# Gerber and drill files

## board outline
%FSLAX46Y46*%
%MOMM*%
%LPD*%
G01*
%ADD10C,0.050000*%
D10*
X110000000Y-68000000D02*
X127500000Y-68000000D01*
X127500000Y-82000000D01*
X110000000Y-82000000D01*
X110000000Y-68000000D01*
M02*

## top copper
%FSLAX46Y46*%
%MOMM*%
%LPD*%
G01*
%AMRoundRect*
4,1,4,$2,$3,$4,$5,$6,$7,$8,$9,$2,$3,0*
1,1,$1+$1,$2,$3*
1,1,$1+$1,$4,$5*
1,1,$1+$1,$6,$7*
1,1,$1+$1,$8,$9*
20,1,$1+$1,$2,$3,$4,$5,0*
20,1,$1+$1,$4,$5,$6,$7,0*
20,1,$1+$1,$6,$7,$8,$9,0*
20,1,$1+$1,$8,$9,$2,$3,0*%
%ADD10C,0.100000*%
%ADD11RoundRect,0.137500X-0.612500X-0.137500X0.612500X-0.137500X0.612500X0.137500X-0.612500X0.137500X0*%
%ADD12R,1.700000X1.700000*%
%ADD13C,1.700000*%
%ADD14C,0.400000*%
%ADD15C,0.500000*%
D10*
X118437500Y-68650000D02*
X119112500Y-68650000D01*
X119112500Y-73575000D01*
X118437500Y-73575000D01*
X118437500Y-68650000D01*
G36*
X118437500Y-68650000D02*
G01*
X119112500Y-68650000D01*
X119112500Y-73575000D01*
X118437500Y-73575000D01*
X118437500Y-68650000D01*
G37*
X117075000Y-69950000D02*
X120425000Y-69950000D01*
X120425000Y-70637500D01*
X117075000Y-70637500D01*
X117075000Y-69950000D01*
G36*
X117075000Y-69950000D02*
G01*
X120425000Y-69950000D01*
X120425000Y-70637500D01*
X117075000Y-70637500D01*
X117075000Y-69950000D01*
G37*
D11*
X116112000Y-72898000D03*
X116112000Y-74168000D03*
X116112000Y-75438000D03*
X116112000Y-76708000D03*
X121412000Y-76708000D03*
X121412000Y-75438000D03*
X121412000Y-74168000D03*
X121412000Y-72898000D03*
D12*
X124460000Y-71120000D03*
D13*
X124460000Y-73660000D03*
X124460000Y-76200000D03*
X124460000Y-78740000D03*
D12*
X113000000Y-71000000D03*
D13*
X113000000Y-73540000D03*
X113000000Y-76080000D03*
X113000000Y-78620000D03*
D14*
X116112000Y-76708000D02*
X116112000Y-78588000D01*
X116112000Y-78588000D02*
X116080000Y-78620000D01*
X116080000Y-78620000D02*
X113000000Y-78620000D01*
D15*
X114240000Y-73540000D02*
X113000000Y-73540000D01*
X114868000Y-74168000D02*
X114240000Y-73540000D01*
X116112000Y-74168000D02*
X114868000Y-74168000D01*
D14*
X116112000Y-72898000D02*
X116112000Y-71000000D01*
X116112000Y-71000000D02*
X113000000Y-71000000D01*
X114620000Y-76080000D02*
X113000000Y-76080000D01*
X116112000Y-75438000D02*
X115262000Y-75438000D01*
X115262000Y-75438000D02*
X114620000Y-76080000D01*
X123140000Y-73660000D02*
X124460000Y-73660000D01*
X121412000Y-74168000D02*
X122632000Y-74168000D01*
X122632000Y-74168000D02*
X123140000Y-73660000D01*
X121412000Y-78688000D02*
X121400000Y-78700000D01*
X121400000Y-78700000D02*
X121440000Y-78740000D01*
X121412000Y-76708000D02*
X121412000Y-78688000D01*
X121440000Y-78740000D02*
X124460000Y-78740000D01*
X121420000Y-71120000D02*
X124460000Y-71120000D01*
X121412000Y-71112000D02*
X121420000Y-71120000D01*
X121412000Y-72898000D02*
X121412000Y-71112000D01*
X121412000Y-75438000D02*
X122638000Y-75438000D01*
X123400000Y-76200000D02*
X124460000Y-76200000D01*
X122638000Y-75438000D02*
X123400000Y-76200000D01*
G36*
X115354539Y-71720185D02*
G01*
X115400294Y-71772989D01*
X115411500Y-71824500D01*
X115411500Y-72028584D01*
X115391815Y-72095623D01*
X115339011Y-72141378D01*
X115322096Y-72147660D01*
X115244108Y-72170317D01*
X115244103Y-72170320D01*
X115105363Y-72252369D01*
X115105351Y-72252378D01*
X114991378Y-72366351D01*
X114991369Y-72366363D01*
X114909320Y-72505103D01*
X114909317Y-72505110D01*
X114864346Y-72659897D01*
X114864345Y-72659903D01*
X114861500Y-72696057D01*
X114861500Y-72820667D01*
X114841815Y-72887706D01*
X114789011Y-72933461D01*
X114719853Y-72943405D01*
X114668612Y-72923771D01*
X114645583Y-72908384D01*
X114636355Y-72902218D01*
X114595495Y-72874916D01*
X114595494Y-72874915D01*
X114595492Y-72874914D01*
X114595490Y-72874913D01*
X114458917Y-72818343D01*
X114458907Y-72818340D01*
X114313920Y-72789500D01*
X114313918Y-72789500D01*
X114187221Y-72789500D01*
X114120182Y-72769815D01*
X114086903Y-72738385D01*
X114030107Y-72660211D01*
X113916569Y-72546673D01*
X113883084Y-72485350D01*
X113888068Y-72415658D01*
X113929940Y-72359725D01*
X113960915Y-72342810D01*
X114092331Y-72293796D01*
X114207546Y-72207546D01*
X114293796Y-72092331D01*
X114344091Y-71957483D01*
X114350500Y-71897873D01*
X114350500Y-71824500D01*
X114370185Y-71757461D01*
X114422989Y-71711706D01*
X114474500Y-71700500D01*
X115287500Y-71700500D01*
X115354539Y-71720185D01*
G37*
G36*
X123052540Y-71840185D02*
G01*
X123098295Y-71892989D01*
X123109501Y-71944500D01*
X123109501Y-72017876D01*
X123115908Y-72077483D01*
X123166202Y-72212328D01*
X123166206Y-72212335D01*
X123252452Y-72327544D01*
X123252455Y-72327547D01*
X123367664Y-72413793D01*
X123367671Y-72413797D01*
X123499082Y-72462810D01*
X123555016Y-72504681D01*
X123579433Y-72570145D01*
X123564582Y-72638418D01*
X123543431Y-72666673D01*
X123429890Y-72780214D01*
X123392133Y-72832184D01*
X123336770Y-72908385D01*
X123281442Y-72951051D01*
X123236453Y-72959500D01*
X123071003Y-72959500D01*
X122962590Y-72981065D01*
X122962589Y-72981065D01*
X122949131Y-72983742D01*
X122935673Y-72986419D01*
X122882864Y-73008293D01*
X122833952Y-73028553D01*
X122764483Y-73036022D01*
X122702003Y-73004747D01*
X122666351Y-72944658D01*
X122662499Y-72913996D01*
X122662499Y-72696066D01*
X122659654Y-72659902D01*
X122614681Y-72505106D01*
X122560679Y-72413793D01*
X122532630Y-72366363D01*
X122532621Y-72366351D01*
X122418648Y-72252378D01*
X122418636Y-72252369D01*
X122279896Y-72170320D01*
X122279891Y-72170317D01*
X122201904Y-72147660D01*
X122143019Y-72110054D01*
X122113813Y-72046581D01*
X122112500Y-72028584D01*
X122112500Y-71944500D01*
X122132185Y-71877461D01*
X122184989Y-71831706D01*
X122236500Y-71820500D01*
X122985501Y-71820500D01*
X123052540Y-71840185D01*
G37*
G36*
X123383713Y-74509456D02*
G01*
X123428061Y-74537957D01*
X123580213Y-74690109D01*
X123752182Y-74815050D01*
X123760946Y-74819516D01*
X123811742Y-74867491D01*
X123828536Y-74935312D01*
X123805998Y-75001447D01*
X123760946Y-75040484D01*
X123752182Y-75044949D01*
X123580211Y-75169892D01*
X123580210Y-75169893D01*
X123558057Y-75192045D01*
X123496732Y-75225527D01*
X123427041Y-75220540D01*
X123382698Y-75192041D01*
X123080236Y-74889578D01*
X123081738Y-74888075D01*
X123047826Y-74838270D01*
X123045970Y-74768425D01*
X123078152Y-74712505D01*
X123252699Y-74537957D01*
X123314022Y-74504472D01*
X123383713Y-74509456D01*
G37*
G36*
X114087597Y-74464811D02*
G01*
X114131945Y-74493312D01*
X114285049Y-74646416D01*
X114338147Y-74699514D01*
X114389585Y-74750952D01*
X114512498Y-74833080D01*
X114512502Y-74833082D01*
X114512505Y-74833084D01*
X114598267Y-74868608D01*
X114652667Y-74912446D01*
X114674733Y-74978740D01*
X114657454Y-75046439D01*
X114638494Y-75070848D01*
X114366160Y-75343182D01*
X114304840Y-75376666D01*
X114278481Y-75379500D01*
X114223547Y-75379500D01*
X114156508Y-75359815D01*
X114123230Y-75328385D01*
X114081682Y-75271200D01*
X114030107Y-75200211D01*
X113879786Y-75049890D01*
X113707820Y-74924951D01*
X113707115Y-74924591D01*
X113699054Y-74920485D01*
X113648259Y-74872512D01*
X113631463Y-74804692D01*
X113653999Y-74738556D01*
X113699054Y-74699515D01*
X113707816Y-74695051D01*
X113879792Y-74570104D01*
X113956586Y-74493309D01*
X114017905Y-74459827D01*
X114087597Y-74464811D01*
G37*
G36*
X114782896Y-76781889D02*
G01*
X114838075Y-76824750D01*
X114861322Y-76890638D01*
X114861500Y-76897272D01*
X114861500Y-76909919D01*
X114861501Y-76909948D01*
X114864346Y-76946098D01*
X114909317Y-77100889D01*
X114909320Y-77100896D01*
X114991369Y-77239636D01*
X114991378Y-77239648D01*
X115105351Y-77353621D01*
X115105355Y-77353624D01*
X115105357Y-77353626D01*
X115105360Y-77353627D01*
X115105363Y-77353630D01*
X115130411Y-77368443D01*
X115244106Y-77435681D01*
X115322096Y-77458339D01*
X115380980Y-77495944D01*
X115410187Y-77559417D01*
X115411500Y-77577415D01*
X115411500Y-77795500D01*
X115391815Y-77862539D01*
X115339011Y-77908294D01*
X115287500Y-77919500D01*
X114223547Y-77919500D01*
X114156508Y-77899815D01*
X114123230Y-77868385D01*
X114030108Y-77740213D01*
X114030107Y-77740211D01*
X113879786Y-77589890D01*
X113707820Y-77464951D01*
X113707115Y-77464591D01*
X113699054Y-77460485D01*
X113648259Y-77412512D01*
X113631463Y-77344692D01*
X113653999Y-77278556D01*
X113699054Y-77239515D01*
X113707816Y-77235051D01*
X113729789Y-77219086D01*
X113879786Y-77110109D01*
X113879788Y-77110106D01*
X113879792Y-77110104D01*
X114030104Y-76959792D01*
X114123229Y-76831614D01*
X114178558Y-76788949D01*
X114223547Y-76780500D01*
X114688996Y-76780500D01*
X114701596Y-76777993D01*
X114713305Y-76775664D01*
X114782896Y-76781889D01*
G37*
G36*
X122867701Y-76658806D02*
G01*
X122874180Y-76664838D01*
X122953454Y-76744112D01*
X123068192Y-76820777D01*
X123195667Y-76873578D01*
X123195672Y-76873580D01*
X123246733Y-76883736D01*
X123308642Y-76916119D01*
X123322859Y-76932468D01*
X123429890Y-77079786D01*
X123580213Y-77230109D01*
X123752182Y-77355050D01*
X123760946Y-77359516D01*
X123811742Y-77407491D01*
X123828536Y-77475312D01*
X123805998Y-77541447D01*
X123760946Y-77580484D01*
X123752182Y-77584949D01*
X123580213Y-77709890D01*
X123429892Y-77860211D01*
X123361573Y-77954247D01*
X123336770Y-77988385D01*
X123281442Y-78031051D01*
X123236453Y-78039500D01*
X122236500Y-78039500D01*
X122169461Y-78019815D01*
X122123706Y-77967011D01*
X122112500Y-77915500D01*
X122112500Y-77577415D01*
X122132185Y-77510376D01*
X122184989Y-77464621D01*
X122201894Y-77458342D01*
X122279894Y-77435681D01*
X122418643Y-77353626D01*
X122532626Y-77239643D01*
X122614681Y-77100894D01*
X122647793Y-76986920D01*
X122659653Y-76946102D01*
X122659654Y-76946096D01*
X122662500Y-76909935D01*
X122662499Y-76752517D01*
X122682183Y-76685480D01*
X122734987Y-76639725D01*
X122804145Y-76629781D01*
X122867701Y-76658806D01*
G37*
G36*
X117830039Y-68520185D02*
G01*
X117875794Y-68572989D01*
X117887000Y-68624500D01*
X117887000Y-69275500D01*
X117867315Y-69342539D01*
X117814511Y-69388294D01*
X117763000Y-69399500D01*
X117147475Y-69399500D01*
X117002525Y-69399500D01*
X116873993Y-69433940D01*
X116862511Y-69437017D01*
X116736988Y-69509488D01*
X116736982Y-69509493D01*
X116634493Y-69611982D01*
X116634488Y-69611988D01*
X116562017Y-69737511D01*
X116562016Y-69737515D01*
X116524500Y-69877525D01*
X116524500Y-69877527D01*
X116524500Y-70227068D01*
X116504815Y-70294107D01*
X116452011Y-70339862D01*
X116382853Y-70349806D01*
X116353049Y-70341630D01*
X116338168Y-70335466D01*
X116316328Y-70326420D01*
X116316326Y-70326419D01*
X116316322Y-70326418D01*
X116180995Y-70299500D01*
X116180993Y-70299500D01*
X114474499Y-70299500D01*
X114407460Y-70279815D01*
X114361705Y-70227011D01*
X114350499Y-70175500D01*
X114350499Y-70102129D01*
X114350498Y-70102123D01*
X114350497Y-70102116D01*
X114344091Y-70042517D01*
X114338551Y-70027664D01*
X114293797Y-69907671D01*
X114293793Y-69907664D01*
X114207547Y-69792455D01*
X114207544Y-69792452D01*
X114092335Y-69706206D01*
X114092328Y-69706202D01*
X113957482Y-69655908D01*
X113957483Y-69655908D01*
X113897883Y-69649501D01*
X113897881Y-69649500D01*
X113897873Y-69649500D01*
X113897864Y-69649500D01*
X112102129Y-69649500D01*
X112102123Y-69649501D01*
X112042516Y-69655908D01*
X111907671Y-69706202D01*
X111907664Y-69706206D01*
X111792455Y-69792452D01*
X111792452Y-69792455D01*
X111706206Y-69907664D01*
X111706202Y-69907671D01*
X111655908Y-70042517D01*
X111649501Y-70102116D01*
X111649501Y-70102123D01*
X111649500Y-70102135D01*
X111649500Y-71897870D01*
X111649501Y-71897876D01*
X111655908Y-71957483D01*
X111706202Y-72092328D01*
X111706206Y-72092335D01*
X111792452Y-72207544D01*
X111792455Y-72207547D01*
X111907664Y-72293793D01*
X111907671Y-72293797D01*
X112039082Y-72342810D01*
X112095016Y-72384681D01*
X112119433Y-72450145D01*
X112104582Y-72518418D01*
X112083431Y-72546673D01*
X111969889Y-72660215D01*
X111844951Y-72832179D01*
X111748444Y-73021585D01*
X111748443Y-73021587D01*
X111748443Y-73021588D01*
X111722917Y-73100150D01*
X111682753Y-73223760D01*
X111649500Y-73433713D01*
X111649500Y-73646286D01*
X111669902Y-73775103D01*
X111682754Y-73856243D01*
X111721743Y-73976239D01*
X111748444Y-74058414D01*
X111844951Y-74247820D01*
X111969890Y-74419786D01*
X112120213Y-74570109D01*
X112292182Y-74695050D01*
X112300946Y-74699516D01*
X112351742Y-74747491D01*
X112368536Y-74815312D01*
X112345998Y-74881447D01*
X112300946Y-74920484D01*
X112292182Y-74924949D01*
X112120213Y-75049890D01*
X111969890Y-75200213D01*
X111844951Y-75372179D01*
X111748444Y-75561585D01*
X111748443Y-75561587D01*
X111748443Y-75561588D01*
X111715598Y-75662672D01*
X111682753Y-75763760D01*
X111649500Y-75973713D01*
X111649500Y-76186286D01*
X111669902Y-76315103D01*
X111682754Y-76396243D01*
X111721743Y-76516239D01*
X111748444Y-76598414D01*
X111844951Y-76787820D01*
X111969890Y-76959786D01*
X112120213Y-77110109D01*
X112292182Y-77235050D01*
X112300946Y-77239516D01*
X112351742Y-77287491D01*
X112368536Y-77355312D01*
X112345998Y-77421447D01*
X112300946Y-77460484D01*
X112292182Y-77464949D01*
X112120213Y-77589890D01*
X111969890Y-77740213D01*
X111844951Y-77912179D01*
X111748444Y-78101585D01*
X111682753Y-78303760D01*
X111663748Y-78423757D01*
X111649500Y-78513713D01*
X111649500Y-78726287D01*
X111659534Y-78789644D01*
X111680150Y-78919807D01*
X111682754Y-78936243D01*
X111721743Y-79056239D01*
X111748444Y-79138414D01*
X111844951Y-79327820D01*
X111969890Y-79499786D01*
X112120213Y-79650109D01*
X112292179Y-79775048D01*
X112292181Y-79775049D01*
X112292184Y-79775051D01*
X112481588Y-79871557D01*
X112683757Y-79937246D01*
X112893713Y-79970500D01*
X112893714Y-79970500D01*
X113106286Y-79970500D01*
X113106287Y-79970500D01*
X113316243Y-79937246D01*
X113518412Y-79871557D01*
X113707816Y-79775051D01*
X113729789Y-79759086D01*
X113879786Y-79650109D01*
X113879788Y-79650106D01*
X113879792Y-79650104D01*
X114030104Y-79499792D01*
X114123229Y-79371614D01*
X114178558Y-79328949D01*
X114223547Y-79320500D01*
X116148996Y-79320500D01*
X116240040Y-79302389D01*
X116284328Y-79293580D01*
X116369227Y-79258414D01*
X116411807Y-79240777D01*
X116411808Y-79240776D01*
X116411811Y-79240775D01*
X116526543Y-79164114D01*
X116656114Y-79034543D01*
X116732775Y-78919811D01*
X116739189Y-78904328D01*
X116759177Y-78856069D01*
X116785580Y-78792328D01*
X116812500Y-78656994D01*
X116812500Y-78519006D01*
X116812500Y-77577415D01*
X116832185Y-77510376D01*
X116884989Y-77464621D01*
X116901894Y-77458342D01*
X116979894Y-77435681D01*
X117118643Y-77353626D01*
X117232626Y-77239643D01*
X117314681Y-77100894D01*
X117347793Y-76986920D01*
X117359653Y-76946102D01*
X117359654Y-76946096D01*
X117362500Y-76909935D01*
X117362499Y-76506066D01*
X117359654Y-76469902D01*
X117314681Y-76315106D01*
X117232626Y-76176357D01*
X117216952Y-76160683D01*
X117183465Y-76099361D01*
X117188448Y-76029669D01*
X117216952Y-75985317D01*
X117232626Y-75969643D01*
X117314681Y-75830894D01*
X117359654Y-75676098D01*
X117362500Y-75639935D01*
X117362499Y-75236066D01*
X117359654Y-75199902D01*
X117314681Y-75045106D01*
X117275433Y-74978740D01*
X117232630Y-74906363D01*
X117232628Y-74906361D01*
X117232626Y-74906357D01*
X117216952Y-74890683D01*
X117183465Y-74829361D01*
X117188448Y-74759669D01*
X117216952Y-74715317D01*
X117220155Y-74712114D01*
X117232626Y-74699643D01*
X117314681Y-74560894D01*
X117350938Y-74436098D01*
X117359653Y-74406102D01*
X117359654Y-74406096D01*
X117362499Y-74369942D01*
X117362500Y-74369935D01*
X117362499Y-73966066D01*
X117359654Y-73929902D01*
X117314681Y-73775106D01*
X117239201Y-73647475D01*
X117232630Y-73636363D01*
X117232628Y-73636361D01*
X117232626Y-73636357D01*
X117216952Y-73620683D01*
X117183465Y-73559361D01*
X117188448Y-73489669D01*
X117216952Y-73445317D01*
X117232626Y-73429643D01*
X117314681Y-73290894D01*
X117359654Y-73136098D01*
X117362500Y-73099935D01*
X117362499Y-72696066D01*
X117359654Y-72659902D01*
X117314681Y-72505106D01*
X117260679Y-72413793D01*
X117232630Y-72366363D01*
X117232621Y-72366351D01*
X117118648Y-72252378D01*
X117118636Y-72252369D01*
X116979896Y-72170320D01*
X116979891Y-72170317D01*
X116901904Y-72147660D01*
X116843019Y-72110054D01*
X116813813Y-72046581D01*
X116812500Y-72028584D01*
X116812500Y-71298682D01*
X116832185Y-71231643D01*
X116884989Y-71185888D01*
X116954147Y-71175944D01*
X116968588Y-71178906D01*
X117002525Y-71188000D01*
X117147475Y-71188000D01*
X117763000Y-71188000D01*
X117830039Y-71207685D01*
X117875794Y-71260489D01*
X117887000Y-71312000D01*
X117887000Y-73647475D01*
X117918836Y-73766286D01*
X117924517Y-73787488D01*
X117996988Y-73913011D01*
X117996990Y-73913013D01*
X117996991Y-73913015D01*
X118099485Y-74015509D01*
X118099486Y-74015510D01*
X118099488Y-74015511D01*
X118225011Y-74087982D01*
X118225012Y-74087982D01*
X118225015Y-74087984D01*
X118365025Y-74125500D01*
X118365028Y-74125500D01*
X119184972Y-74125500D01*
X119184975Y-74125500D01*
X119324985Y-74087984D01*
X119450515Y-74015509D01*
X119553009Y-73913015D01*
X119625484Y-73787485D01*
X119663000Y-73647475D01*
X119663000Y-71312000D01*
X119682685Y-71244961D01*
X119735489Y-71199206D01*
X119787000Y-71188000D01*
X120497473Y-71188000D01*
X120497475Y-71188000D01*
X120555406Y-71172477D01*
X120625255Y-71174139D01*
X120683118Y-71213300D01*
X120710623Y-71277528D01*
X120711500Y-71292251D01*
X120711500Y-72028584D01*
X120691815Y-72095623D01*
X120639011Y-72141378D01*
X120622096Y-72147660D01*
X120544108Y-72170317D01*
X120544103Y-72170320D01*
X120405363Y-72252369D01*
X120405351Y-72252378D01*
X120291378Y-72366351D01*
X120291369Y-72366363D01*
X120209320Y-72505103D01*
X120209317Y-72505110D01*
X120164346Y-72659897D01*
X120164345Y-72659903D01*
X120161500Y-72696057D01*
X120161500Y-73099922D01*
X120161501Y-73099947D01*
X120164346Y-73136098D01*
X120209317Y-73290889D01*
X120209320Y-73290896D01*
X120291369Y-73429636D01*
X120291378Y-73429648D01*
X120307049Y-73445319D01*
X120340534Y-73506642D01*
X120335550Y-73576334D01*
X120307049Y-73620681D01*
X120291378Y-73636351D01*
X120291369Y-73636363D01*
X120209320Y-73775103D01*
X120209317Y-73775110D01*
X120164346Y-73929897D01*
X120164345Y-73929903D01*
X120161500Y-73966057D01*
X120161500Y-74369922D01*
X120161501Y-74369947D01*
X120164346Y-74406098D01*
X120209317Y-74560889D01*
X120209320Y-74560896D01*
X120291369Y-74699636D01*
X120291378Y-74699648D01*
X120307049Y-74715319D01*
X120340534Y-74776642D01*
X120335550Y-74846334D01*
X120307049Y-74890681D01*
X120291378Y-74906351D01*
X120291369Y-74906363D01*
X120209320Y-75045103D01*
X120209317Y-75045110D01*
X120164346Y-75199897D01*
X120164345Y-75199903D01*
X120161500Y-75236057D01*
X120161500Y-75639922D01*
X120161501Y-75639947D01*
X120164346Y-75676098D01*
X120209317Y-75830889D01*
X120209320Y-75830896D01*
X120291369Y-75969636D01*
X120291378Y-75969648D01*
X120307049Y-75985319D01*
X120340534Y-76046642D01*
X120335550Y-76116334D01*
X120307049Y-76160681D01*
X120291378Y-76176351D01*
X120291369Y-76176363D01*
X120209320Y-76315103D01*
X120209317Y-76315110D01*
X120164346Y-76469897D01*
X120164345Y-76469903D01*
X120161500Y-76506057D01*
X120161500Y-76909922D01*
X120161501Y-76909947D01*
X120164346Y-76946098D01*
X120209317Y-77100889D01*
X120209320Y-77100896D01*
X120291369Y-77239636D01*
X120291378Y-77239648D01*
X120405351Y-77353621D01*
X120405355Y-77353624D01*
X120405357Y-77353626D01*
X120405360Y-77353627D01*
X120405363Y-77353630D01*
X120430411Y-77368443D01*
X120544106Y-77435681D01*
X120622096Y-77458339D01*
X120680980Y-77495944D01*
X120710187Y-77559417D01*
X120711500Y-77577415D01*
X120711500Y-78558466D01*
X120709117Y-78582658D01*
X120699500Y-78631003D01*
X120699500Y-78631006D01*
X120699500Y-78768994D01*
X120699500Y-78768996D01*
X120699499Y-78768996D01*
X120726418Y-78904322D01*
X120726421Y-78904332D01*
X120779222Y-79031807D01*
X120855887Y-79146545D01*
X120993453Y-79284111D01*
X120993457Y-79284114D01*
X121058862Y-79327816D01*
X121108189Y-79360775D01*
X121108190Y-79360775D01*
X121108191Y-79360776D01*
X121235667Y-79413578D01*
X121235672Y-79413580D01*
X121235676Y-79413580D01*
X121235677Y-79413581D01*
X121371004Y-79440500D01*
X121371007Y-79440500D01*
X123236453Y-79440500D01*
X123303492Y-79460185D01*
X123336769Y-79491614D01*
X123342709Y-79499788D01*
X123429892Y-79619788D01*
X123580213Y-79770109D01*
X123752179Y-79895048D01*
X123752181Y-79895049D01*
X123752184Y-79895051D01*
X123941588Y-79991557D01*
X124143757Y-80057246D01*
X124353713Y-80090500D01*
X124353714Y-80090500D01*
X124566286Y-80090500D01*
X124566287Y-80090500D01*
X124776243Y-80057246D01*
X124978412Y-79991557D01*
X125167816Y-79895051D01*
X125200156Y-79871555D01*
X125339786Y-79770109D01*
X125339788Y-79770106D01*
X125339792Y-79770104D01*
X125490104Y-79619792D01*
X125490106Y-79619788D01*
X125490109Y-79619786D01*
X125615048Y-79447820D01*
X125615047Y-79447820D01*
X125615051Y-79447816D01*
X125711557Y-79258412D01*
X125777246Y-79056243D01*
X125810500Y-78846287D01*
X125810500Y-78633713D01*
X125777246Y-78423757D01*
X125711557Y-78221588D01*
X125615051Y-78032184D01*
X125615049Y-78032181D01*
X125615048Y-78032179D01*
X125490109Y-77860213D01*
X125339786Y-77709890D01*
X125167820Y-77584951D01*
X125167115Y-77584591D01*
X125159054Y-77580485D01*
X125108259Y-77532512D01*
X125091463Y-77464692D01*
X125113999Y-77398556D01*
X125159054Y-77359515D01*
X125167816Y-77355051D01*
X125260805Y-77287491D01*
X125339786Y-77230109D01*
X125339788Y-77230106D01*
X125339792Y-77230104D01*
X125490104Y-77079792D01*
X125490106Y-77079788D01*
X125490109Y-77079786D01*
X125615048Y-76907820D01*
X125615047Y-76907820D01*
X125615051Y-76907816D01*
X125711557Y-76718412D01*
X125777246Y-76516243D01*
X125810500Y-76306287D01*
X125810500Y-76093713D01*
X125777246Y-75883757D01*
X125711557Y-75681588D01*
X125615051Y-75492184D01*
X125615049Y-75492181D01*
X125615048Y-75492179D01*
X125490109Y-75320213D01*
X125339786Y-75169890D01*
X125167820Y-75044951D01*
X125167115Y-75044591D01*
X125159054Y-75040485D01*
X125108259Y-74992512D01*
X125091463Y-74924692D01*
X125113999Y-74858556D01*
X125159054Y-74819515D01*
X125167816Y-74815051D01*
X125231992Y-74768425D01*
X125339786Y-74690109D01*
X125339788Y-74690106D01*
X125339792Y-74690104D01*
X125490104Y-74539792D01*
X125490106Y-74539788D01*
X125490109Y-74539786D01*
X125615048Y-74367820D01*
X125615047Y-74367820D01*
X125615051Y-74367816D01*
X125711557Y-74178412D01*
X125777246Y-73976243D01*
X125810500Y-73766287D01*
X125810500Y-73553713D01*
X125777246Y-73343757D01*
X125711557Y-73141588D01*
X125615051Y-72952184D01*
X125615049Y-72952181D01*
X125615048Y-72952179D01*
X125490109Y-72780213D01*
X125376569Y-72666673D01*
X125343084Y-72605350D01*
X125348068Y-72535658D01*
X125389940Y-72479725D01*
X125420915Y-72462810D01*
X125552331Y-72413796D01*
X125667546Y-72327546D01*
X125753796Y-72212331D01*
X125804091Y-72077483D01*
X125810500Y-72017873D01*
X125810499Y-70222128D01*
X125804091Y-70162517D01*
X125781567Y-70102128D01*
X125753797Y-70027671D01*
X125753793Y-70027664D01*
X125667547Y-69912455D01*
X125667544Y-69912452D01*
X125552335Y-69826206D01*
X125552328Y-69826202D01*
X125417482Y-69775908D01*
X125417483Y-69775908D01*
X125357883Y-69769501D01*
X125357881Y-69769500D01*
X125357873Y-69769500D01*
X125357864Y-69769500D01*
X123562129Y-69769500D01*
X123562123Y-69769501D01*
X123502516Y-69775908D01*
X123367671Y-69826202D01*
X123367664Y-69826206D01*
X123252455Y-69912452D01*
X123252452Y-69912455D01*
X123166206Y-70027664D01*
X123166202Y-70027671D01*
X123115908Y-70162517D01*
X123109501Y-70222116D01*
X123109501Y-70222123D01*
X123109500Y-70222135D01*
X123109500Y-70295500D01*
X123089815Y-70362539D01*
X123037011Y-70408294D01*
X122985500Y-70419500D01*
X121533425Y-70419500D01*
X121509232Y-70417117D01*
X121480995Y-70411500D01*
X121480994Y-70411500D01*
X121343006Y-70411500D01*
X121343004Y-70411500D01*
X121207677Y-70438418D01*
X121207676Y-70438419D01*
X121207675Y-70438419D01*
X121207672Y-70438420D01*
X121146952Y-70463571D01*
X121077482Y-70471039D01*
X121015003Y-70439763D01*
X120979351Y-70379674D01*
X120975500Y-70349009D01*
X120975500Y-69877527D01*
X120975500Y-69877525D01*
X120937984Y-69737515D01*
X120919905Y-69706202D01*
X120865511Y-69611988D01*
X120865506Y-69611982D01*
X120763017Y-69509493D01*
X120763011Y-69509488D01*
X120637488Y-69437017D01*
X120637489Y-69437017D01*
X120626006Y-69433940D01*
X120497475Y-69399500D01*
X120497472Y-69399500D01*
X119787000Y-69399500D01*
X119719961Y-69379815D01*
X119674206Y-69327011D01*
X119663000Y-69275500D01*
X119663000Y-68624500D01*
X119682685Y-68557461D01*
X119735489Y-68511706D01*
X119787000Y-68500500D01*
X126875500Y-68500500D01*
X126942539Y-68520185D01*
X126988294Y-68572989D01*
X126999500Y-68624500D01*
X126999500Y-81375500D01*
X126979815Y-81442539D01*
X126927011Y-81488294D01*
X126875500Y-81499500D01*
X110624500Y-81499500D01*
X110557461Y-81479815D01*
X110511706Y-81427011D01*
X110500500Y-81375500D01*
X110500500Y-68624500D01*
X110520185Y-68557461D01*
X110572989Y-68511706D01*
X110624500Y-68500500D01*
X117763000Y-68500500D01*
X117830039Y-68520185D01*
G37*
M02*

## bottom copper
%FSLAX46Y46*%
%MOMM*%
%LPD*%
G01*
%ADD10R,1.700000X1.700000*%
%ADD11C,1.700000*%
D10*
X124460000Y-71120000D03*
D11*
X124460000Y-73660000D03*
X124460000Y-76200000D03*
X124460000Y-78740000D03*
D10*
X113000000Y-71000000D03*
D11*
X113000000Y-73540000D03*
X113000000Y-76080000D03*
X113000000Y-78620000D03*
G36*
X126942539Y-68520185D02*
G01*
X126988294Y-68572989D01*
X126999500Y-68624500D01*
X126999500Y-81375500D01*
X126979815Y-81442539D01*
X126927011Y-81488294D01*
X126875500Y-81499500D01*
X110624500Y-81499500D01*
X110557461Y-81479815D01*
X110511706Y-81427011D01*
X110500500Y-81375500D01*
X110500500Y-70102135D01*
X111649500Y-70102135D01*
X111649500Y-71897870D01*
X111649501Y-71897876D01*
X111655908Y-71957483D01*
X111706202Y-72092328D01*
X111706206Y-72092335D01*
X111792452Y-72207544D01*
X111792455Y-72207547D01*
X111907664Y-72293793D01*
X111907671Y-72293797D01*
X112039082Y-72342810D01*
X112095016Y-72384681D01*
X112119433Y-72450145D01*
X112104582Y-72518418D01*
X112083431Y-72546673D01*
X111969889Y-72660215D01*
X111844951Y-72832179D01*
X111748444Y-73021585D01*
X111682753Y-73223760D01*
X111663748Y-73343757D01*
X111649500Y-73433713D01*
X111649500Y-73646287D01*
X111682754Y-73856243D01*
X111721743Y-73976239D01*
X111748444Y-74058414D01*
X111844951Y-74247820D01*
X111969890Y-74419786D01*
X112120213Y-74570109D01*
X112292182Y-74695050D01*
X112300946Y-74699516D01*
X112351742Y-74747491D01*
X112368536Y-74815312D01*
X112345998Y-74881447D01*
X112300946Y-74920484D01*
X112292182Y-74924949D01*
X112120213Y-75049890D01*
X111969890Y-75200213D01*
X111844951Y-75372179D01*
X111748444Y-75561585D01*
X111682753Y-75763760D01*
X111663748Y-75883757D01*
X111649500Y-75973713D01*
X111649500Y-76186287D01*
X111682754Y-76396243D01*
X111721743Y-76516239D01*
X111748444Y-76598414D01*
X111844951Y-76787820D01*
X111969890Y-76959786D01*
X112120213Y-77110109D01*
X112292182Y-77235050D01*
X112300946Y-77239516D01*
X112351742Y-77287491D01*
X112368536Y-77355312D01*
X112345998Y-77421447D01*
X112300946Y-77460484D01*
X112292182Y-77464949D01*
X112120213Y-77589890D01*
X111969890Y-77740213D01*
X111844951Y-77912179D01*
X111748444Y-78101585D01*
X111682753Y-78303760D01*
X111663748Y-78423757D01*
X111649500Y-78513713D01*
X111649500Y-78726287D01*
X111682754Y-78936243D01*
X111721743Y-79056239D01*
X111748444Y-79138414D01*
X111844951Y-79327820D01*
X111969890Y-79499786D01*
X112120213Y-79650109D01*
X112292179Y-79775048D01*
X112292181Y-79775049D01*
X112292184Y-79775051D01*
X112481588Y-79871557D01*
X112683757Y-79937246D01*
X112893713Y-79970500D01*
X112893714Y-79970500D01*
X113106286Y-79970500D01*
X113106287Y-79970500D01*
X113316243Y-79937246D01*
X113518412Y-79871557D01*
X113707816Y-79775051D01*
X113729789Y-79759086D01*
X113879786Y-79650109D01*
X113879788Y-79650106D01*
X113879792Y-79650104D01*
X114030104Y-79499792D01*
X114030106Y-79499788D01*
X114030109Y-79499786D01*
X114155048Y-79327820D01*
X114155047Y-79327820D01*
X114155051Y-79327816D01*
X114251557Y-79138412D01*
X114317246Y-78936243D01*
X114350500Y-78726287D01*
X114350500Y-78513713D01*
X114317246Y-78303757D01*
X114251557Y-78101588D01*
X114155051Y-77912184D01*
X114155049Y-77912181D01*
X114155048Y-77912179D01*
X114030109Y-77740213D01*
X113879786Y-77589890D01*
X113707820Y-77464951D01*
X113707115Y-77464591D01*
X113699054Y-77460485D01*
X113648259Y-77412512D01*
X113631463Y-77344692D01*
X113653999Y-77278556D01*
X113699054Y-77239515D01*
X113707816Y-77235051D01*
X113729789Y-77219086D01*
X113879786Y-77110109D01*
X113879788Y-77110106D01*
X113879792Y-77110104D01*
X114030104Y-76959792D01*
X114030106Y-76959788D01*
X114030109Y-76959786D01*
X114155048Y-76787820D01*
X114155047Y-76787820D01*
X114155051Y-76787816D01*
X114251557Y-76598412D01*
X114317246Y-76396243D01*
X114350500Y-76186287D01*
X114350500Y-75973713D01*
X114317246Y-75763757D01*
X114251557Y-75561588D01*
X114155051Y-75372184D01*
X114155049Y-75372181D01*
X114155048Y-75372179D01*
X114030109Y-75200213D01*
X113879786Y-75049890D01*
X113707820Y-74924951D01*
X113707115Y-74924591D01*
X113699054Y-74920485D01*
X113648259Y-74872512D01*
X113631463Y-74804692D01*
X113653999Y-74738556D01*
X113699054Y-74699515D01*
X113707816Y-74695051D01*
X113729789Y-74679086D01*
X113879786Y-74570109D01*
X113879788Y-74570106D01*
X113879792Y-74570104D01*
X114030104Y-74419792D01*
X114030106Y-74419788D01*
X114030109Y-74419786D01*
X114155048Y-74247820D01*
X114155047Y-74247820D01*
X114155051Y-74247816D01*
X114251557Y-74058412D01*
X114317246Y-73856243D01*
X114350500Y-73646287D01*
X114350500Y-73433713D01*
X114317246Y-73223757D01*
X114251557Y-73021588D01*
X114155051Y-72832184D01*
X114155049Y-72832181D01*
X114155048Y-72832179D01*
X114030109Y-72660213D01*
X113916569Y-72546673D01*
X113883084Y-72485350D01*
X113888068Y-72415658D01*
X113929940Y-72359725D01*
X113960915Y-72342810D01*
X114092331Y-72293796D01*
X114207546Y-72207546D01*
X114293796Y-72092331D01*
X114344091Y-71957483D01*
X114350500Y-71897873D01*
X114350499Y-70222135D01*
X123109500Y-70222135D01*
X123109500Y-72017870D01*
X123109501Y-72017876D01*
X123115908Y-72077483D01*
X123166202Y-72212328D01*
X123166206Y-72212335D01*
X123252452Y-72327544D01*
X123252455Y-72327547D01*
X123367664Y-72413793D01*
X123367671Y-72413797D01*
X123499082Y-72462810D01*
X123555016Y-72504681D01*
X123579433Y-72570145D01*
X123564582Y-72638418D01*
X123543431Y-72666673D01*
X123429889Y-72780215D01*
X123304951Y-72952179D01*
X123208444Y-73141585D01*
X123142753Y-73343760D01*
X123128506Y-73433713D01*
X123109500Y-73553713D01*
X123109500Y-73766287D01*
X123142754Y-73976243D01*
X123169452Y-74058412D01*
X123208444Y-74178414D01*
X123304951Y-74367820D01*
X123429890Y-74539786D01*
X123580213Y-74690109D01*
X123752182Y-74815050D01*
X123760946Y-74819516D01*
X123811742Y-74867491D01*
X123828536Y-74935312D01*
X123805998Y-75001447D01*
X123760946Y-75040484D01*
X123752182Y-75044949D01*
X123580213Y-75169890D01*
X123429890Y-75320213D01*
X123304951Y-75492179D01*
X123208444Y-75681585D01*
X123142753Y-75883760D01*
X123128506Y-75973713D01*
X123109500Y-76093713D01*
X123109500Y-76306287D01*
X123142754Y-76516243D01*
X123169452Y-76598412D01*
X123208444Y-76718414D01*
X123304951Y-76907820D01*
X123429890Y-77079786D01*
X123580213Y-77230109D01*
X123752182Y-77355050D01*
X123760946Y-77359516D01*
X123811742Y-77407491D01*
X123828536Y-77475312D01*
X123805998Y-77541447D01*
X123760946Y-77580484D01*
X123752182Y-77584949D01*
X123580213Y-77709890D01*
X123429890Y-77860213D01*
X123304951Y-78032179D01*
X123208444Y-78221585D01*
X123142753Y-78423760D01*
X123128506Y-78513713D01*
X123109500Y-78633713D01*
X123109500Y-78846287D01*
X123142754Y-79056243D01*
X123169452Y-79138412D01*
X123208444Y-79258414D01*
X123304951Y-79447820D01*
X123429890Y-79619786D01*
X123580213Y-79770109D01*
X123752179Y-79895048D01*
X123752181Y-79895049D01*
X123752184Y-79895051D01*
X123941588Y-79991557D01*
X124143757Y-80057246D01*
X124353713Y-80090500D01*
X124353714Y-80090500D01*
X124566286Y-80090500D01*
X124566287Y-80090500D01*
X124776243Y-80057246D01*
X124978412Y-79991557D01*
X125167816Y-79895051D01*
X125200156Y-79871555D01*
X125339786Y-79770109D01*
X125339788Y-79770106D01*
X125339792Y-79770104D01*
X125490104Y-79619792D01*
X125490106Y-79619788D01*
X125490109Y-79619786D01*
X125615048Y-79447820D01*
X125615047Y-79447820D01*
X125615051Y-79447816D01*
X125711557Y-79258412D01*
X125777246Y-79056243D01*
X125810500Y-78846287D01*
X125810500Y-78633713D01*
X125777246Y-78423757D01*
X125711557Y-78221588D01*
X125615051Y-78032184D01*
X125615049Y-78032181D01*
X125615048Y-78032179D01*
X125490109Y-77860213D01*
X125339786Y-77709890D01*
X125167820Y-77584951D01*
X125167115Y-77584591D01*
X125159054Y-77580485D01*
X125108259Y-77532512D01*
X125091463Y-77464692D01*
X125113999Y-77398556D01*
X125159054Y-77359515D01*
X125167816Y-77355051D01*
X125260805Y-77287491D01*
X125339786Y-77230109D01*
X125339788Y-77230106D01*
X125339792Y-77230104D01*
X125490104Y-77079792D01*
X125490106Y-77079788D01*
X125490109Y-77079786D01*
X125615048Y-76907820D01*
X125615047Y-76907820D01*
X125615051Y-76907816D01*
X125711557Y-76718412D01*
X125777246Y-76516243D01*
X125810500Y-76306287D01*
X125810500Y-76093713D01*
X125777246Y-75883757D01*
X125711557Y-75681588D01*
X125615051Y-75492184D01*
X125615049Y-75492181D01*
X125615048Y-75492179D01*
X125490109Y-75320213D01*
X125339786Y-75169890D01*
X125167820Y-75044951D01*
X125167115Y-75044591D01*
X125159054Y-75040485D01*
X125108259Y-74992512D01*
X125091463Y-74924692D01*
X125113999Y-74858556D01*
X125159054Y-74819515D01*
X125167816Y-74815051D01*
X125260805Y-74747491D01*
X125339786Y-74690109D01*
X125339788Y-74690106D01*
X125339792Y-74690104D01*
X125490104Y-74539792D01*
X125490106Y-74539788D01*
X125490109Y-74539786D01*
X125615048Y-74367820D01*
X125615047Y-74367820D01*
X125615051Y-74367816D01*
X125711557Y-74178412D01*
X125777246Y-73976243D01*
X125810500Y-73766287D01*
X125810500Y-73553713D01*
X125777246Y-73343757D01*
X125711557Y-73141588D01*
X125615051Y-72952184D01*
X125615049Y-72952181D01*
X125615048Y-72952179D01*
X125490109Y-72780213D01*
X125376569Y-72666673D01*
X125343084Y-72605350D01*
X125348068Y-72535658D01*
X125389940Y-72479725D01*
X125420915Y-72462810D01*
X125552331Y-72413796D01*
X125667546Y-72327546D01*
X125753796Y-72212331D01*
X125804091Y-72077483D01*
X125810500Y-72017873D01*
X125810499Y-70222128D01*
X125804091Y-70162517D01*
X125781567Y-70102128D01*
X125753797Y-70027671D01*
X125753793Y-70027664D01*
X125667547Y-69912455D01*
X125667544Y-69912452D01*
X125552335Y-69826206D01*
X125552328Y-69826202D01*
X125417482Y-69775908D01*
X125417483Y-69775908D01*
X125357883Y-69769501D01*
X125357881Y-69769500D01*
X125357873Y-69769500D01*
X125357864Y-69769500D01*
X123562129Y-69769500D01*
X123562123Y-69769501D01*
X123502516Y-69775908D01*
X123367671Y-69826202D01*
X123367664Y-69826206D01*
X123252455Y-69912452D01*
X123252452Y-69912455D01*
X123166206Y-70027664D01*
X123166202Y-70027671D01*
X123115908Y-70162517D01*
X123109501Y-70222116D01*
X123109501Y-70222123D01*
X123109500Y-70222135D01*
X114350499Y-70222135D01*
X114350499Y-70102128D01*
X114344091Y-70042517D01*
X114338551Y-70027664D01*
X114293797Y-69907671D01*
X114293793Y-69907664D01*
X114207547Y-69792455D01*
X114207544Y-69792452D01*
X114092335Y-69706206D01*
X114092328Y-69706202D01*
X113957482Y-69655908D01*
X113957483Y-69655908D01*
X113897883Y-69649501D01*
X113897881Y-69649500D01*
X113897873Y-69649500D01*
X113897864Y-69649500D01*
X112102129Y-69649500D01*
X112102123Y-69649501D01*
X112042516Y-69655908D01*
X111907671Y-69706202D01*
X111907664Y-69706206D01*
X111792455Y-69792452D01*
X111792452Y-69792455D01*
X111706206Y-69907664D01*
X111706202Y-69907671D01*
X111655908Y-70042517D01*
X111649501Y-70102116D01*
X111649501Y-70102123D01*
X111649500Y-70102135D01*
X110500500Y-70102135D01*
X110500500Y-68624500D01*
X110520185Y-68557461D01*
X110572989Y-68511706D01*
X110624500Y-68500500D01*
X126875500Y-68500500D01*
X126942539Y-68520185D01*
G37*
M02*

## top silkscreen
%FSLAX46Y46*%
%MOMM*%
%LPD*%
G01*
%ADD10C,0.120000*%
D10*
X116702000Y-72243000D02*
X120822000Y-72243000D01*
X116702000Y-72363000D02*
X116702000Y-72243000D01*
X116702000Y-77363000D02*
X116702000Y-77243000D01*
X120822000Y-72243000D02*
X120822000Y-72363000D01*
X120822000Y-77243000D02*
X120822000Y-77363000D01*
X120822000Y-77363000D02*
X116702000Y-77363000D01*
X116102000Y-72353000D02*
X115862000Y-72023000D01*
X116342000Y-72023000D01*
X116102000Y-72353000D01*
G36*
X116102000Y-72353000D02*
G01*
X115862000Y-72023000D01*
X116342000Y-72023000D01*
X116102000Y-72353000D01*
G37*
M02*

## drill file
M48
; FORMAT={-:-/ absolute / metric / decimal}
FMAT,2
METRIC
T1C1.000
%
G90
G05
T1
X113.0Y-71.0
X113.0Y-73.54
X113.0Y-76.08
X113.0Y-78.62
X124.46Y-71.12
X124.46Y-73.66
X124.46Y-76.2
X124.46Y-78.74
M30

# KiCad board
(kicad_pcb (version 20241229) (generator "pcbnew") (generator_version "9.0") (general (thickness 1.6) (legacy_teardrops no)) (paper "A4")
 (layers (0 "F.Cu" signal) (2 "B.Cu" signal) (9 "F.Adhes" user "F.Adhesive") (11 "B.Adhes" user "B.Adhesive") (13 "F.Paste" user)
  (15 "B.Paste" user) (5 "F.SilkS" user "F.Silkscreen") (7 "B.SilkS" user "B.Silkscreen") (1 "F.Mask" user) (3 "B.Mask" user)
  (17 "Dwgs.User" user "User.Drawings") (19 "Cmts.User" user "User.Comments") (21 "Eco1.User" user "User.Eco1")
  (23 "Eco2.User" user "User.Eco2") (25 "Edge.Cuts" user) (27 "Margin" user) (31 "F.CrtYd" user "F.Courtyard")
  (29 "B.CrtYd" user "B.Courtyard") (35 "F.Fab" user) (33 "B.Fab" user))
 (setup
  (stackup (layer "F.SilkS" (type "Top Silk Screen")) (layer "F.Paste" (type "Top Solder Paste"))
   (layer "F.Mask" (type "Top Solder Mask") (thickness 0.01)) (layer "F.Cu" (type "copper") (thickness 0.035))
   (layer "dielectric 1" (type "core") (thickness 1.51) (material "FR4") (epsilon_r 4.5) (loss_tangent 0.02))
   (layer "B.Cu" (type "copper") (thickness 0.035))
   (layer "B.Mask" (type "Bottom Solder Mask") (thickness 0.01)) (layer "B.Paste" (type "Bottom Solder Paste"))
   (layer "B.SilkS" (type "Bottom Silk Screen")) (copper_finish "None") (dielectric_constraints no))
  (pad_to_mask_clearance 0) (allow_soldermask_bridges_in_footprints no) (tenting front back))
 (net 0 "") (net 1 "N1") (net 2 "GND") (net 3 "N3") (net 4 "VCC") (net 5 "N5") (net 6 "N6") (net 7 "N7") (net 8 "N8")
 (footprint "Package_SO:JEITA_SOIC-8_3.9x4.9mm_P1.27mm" (layer "F.Cu") (at 118.762 74.803)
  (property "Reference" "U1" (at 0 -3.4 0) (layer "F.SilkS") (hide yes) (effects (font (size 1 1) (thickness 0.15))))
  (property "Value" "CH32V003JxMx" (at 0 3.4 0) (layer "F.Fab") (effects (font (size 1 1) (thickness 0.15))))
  (fp_line (start -2.06 -2.56) (end 2.06 -2.56) (stroke (width 0.12) (type solid)) (layer "F.SilkS"))
  (fp_line (start -2.06 -2.44) (end -2.06 -2.56) (stroke (width 0.12) (type solid)) (layer "F.SilkS"))
  (fp_line (start -2.06 2.56) (end -2.06 2.44) (stroke (width 0.12) (type solid)) (layer "F.SilkS"))
  (fp_line (start 2.06 -2.56) (end 2.06 -2.44) (stroke (width 0.12) (type solid)) (layer "F.SilkS"))
  (fp_line (start 2.06 2.44) (end 2.06 2.56) (stroke (width 0.12) (type solid)) (layer "F.SilkS"))
  (fp_line (start 2.06 2.56) (end -2.06 2.56) (stroke (width 0.12) (type solid)) (layer "F.SilkS"))
  (fp_poly (pts (xy -2.66 -2.45) (xy -2.9 -2.78) (xy -2.42 -2.78)) (stroke (width 0.12) (type solid)) (fill yes) (layer "F.SilkS"))
  (pad "1" smd roundrect (at -2.65 -1.905) (size 1.5 0.55) (layers "F.Cu" "F.Mask" "F.Paste") (roundrect_rratio 0.25) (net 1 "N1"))
  (pad "2" smd roundrect (at -2.65 -0.635) (size 1.5 0.55) (layers "F.Cu" "F.Mask" "F.Paste") (roundrect_rratio 0.25) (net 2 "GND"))
  (pad "3" smd roundrect (at -2.65 0.635) (size 1.5 0.55) (layers "F.Cu" "F.Mask" "F.Paste") (roundrect_rratio 0.25) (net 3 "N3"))
  (pad "4" smd roundrect (at -2.65 1.905) (size 1.5 0.55) (layers "F.Cu" "F.Mask" "F.Paste") (roundrect_rratio 0.25) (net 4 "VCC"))
  (pad "5" smd roundrect (at 2.65 1.905) (size 1.5 0.55) (layers "F.Cu" "F.Mask" "F.Paste") (roundrect_rratio 0.25) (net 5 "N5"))
  (pad "6" smd roundrect (at 2.65 0.635) (size 1.5 0.55) (layers "F.Cu" "F.Mask" "F.Paste") (roundrect_rratio 0.25) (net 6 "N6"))
  (pad "7" smd roundrect (at 2.65 -0.635) (size 1.5 0.55) (layers "F.Cu" "F.Mask" "F.Paste") (roundrect_rratio 0.25) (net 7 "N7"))
  (pad "8" smd roundrect (at 2.65 -1.905) (size 1.5 0.55) (layers "F.Cu" "F.Mask" "F.Paste") (roundrect_rratio 0.25) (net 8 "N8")))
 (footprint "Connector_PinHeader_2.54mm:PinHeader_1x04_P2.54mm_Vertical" (layer "B.Cu") (at 124.46 71.12 180)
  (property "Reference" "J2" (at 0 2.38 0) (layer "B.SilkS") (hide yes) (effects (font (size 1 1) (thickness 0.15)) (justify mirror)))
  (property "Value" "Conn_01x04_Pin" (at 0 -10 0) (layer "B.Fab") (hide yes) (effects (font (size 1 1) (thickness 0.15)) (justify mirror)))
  (pad "1" thru_hole rect (at 0 0 180) (size 1.7 1.7) (drill 1) (layers "*.Cu" "*.Mask") (remove_unused_layers no) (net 8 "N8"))
  (pad "2" thru_hole circle (at 0 -2.54 180) (size 1.7 1.7) (drill 1) (layers "*.Cu" "*.Mask") (remove_unused_layers no) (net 7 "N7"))
  (pad "3" thru_hole circle (at 0 -5.08 180) (size 1.7 1.7) (drill 1) (layers "*.Cu" "*.Mask") (remove_unused_layers no) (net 6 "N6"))
  (pad "4" thru_hole circle (at 0 -7.62 180) (size 1.7 1.7) (drill 1) (layers "*.Cu" "*.Mask") (remove_unused_layers no) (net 5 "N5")))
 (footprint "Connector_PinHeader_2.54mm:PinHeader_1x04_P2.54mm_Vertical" (layer "B.Cu") (at 113 71 180)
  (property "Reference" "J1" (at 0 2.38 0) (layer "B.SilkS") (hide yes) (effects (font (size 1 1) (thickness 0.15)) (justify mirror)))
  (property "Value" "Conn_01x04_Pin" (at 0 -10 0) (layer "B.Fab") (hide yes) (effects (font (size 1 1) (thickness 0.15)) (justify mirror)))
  (pad "1" thru_hole rect (at 0 0 180) (size 1.7 1.7) (drill 1) (layers "*.Cu" "*.Mask") (remove_unused_layers no) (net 1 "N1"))
  (pad "2" thru_hole circle (at 0 -2.54 180) (size 1.7 1.7) (drill 1) (layers "*.Cu" "*.Mask") (remove_unused_layers no) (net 2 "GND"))
  (pad "3" thru_hole circle (at 0 -5.08 180) (size 1.7 1.7) (drill 1) (layers "*.Cu" "*.Mask") (remove_unused_layers no) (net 3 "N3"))
  (pad "4" thru_hole circle (at 0 -7.62 180) (size 1.7 1.7) (drill 1) (layers "*.Cu" "*.Mask") (remove_unused_layers no) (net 4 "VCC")))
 (gr_rect (start 118.4375 68.65) (end 119.1125 73.575) (stroke (width 0.1) (type solid)) (fill yes) (layer "F.Cu"))
 (gr_rect (start 117.075 69.95) (end 120.425 70.6375) (stroke (width 0.1) (type solid)) (fill yes) (layer "F.Cu"))
 (gr_rect (start 110 68) (end 127.5 82) (stroke (width 0.05) (type default)) (fill no) (layer "Edge.Cuts"))
 (segment (start 116.112 76.708) (end 116.112 78.588) (width 0.4) (layer "F.Cu") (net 4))
 (segment (start 116.112 78.588) (end 116.08 78.62) (width 0.4) (layer "F.Cu") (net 4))
 (segment (start 116.08 78.62) (end 113 78.62) (width 0.4) (layer "F.Cu") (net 4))
 (segment (start 114.24 73.54) (end 113 73.54) (width 0.5) (layer "F.Cu") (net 2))
 (segment (start 114.868 74.168) (end 114.24 73.54) (width 0.5) (layer "F.Cu") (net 2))
 (segment (start 116.112 74.168) (end 114.868 74.168) (width 0.5) (layer "F.Cu") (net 2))
 (segment (start 116.112 72.898) (end 116.112 71) (width 0.4) (layer "F.Cu") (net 1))
 (segment (start 116.112 71) (end 113 71) (width 0.4) (layer "F.Cu") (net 1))
 (segment (start 114.62 76.08) (end 113 76.08) (width 0.4) (layer "F.Cu") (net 3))
 (segment (start 116.112 75.438) (end 115.262 75.438) (width 0.4) (layer "F.Cu") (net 3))
 (segment (start 115.262 75.438) (end 114.62 76.08) (width 0.4) (layer "F.Cu") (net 3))
 (segment (start 123.14 73.66) (end 124.46 73.66) (width 0.4) (layer "F.Cu") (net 7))
 (segment (start 121.412 74.168) (end 122.632 74.168) (width 0.4) (layer "F.Cu") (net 7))
 (segment (start 122.632 74.168) (end 123.14 73.66) (width 0.4) (layer "F.Cu") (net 7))
 (segment (start 121.412 78.688) (end 121.4 78.7) (width 0.4) (layer "F.Cu") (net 5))
 (segment (start 121.4 78.7) (end 121.44 78.74) (width 0.4) (layer "F.Cu") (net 5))
 (segment (start 121.412 76.708) (end 121.412 78.688) (width 0.4) (layer "F.Cu") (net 5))
 (segment (start 121.44 78.74) (end 124.46 78.74) (width 0.4) (layer "F.Cu") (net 5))
 (segment (start 121.42 71.12) (end 124.46 71.12) (width 0.4) (layer "F.Cu") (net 8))
 (segment (start 121.412 71.112) (end 121.42 71.12) (width 0.4) (layer "F.Cu") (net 8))
 (segment (start 121.412 72.898) (end 121.412 71.112) (width 0.4) (layer "F.Cu") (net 8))
 (segment (start 121.412 75.438) (end 122.638 75.438) (width 0.4) (layer "F.Cu") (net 6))
 (segment (start 123.4 76.2) (end 124.46 76.2) (width 0.4) (layer "F.Cu") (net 6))
 (segment (start 122.638 75.438) (end 123.4 76.2) (width 0.4) (layer "F.Cu") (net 6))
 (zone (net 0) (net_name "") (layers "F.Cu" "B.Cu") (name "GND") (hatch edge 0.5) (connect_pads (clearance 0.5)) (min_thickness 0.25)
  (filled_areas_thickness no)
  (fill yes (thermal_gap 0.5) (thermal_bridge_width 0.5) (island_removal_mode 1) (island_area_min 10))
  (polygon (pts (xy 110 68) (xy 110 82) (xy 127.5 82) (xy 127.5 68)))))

